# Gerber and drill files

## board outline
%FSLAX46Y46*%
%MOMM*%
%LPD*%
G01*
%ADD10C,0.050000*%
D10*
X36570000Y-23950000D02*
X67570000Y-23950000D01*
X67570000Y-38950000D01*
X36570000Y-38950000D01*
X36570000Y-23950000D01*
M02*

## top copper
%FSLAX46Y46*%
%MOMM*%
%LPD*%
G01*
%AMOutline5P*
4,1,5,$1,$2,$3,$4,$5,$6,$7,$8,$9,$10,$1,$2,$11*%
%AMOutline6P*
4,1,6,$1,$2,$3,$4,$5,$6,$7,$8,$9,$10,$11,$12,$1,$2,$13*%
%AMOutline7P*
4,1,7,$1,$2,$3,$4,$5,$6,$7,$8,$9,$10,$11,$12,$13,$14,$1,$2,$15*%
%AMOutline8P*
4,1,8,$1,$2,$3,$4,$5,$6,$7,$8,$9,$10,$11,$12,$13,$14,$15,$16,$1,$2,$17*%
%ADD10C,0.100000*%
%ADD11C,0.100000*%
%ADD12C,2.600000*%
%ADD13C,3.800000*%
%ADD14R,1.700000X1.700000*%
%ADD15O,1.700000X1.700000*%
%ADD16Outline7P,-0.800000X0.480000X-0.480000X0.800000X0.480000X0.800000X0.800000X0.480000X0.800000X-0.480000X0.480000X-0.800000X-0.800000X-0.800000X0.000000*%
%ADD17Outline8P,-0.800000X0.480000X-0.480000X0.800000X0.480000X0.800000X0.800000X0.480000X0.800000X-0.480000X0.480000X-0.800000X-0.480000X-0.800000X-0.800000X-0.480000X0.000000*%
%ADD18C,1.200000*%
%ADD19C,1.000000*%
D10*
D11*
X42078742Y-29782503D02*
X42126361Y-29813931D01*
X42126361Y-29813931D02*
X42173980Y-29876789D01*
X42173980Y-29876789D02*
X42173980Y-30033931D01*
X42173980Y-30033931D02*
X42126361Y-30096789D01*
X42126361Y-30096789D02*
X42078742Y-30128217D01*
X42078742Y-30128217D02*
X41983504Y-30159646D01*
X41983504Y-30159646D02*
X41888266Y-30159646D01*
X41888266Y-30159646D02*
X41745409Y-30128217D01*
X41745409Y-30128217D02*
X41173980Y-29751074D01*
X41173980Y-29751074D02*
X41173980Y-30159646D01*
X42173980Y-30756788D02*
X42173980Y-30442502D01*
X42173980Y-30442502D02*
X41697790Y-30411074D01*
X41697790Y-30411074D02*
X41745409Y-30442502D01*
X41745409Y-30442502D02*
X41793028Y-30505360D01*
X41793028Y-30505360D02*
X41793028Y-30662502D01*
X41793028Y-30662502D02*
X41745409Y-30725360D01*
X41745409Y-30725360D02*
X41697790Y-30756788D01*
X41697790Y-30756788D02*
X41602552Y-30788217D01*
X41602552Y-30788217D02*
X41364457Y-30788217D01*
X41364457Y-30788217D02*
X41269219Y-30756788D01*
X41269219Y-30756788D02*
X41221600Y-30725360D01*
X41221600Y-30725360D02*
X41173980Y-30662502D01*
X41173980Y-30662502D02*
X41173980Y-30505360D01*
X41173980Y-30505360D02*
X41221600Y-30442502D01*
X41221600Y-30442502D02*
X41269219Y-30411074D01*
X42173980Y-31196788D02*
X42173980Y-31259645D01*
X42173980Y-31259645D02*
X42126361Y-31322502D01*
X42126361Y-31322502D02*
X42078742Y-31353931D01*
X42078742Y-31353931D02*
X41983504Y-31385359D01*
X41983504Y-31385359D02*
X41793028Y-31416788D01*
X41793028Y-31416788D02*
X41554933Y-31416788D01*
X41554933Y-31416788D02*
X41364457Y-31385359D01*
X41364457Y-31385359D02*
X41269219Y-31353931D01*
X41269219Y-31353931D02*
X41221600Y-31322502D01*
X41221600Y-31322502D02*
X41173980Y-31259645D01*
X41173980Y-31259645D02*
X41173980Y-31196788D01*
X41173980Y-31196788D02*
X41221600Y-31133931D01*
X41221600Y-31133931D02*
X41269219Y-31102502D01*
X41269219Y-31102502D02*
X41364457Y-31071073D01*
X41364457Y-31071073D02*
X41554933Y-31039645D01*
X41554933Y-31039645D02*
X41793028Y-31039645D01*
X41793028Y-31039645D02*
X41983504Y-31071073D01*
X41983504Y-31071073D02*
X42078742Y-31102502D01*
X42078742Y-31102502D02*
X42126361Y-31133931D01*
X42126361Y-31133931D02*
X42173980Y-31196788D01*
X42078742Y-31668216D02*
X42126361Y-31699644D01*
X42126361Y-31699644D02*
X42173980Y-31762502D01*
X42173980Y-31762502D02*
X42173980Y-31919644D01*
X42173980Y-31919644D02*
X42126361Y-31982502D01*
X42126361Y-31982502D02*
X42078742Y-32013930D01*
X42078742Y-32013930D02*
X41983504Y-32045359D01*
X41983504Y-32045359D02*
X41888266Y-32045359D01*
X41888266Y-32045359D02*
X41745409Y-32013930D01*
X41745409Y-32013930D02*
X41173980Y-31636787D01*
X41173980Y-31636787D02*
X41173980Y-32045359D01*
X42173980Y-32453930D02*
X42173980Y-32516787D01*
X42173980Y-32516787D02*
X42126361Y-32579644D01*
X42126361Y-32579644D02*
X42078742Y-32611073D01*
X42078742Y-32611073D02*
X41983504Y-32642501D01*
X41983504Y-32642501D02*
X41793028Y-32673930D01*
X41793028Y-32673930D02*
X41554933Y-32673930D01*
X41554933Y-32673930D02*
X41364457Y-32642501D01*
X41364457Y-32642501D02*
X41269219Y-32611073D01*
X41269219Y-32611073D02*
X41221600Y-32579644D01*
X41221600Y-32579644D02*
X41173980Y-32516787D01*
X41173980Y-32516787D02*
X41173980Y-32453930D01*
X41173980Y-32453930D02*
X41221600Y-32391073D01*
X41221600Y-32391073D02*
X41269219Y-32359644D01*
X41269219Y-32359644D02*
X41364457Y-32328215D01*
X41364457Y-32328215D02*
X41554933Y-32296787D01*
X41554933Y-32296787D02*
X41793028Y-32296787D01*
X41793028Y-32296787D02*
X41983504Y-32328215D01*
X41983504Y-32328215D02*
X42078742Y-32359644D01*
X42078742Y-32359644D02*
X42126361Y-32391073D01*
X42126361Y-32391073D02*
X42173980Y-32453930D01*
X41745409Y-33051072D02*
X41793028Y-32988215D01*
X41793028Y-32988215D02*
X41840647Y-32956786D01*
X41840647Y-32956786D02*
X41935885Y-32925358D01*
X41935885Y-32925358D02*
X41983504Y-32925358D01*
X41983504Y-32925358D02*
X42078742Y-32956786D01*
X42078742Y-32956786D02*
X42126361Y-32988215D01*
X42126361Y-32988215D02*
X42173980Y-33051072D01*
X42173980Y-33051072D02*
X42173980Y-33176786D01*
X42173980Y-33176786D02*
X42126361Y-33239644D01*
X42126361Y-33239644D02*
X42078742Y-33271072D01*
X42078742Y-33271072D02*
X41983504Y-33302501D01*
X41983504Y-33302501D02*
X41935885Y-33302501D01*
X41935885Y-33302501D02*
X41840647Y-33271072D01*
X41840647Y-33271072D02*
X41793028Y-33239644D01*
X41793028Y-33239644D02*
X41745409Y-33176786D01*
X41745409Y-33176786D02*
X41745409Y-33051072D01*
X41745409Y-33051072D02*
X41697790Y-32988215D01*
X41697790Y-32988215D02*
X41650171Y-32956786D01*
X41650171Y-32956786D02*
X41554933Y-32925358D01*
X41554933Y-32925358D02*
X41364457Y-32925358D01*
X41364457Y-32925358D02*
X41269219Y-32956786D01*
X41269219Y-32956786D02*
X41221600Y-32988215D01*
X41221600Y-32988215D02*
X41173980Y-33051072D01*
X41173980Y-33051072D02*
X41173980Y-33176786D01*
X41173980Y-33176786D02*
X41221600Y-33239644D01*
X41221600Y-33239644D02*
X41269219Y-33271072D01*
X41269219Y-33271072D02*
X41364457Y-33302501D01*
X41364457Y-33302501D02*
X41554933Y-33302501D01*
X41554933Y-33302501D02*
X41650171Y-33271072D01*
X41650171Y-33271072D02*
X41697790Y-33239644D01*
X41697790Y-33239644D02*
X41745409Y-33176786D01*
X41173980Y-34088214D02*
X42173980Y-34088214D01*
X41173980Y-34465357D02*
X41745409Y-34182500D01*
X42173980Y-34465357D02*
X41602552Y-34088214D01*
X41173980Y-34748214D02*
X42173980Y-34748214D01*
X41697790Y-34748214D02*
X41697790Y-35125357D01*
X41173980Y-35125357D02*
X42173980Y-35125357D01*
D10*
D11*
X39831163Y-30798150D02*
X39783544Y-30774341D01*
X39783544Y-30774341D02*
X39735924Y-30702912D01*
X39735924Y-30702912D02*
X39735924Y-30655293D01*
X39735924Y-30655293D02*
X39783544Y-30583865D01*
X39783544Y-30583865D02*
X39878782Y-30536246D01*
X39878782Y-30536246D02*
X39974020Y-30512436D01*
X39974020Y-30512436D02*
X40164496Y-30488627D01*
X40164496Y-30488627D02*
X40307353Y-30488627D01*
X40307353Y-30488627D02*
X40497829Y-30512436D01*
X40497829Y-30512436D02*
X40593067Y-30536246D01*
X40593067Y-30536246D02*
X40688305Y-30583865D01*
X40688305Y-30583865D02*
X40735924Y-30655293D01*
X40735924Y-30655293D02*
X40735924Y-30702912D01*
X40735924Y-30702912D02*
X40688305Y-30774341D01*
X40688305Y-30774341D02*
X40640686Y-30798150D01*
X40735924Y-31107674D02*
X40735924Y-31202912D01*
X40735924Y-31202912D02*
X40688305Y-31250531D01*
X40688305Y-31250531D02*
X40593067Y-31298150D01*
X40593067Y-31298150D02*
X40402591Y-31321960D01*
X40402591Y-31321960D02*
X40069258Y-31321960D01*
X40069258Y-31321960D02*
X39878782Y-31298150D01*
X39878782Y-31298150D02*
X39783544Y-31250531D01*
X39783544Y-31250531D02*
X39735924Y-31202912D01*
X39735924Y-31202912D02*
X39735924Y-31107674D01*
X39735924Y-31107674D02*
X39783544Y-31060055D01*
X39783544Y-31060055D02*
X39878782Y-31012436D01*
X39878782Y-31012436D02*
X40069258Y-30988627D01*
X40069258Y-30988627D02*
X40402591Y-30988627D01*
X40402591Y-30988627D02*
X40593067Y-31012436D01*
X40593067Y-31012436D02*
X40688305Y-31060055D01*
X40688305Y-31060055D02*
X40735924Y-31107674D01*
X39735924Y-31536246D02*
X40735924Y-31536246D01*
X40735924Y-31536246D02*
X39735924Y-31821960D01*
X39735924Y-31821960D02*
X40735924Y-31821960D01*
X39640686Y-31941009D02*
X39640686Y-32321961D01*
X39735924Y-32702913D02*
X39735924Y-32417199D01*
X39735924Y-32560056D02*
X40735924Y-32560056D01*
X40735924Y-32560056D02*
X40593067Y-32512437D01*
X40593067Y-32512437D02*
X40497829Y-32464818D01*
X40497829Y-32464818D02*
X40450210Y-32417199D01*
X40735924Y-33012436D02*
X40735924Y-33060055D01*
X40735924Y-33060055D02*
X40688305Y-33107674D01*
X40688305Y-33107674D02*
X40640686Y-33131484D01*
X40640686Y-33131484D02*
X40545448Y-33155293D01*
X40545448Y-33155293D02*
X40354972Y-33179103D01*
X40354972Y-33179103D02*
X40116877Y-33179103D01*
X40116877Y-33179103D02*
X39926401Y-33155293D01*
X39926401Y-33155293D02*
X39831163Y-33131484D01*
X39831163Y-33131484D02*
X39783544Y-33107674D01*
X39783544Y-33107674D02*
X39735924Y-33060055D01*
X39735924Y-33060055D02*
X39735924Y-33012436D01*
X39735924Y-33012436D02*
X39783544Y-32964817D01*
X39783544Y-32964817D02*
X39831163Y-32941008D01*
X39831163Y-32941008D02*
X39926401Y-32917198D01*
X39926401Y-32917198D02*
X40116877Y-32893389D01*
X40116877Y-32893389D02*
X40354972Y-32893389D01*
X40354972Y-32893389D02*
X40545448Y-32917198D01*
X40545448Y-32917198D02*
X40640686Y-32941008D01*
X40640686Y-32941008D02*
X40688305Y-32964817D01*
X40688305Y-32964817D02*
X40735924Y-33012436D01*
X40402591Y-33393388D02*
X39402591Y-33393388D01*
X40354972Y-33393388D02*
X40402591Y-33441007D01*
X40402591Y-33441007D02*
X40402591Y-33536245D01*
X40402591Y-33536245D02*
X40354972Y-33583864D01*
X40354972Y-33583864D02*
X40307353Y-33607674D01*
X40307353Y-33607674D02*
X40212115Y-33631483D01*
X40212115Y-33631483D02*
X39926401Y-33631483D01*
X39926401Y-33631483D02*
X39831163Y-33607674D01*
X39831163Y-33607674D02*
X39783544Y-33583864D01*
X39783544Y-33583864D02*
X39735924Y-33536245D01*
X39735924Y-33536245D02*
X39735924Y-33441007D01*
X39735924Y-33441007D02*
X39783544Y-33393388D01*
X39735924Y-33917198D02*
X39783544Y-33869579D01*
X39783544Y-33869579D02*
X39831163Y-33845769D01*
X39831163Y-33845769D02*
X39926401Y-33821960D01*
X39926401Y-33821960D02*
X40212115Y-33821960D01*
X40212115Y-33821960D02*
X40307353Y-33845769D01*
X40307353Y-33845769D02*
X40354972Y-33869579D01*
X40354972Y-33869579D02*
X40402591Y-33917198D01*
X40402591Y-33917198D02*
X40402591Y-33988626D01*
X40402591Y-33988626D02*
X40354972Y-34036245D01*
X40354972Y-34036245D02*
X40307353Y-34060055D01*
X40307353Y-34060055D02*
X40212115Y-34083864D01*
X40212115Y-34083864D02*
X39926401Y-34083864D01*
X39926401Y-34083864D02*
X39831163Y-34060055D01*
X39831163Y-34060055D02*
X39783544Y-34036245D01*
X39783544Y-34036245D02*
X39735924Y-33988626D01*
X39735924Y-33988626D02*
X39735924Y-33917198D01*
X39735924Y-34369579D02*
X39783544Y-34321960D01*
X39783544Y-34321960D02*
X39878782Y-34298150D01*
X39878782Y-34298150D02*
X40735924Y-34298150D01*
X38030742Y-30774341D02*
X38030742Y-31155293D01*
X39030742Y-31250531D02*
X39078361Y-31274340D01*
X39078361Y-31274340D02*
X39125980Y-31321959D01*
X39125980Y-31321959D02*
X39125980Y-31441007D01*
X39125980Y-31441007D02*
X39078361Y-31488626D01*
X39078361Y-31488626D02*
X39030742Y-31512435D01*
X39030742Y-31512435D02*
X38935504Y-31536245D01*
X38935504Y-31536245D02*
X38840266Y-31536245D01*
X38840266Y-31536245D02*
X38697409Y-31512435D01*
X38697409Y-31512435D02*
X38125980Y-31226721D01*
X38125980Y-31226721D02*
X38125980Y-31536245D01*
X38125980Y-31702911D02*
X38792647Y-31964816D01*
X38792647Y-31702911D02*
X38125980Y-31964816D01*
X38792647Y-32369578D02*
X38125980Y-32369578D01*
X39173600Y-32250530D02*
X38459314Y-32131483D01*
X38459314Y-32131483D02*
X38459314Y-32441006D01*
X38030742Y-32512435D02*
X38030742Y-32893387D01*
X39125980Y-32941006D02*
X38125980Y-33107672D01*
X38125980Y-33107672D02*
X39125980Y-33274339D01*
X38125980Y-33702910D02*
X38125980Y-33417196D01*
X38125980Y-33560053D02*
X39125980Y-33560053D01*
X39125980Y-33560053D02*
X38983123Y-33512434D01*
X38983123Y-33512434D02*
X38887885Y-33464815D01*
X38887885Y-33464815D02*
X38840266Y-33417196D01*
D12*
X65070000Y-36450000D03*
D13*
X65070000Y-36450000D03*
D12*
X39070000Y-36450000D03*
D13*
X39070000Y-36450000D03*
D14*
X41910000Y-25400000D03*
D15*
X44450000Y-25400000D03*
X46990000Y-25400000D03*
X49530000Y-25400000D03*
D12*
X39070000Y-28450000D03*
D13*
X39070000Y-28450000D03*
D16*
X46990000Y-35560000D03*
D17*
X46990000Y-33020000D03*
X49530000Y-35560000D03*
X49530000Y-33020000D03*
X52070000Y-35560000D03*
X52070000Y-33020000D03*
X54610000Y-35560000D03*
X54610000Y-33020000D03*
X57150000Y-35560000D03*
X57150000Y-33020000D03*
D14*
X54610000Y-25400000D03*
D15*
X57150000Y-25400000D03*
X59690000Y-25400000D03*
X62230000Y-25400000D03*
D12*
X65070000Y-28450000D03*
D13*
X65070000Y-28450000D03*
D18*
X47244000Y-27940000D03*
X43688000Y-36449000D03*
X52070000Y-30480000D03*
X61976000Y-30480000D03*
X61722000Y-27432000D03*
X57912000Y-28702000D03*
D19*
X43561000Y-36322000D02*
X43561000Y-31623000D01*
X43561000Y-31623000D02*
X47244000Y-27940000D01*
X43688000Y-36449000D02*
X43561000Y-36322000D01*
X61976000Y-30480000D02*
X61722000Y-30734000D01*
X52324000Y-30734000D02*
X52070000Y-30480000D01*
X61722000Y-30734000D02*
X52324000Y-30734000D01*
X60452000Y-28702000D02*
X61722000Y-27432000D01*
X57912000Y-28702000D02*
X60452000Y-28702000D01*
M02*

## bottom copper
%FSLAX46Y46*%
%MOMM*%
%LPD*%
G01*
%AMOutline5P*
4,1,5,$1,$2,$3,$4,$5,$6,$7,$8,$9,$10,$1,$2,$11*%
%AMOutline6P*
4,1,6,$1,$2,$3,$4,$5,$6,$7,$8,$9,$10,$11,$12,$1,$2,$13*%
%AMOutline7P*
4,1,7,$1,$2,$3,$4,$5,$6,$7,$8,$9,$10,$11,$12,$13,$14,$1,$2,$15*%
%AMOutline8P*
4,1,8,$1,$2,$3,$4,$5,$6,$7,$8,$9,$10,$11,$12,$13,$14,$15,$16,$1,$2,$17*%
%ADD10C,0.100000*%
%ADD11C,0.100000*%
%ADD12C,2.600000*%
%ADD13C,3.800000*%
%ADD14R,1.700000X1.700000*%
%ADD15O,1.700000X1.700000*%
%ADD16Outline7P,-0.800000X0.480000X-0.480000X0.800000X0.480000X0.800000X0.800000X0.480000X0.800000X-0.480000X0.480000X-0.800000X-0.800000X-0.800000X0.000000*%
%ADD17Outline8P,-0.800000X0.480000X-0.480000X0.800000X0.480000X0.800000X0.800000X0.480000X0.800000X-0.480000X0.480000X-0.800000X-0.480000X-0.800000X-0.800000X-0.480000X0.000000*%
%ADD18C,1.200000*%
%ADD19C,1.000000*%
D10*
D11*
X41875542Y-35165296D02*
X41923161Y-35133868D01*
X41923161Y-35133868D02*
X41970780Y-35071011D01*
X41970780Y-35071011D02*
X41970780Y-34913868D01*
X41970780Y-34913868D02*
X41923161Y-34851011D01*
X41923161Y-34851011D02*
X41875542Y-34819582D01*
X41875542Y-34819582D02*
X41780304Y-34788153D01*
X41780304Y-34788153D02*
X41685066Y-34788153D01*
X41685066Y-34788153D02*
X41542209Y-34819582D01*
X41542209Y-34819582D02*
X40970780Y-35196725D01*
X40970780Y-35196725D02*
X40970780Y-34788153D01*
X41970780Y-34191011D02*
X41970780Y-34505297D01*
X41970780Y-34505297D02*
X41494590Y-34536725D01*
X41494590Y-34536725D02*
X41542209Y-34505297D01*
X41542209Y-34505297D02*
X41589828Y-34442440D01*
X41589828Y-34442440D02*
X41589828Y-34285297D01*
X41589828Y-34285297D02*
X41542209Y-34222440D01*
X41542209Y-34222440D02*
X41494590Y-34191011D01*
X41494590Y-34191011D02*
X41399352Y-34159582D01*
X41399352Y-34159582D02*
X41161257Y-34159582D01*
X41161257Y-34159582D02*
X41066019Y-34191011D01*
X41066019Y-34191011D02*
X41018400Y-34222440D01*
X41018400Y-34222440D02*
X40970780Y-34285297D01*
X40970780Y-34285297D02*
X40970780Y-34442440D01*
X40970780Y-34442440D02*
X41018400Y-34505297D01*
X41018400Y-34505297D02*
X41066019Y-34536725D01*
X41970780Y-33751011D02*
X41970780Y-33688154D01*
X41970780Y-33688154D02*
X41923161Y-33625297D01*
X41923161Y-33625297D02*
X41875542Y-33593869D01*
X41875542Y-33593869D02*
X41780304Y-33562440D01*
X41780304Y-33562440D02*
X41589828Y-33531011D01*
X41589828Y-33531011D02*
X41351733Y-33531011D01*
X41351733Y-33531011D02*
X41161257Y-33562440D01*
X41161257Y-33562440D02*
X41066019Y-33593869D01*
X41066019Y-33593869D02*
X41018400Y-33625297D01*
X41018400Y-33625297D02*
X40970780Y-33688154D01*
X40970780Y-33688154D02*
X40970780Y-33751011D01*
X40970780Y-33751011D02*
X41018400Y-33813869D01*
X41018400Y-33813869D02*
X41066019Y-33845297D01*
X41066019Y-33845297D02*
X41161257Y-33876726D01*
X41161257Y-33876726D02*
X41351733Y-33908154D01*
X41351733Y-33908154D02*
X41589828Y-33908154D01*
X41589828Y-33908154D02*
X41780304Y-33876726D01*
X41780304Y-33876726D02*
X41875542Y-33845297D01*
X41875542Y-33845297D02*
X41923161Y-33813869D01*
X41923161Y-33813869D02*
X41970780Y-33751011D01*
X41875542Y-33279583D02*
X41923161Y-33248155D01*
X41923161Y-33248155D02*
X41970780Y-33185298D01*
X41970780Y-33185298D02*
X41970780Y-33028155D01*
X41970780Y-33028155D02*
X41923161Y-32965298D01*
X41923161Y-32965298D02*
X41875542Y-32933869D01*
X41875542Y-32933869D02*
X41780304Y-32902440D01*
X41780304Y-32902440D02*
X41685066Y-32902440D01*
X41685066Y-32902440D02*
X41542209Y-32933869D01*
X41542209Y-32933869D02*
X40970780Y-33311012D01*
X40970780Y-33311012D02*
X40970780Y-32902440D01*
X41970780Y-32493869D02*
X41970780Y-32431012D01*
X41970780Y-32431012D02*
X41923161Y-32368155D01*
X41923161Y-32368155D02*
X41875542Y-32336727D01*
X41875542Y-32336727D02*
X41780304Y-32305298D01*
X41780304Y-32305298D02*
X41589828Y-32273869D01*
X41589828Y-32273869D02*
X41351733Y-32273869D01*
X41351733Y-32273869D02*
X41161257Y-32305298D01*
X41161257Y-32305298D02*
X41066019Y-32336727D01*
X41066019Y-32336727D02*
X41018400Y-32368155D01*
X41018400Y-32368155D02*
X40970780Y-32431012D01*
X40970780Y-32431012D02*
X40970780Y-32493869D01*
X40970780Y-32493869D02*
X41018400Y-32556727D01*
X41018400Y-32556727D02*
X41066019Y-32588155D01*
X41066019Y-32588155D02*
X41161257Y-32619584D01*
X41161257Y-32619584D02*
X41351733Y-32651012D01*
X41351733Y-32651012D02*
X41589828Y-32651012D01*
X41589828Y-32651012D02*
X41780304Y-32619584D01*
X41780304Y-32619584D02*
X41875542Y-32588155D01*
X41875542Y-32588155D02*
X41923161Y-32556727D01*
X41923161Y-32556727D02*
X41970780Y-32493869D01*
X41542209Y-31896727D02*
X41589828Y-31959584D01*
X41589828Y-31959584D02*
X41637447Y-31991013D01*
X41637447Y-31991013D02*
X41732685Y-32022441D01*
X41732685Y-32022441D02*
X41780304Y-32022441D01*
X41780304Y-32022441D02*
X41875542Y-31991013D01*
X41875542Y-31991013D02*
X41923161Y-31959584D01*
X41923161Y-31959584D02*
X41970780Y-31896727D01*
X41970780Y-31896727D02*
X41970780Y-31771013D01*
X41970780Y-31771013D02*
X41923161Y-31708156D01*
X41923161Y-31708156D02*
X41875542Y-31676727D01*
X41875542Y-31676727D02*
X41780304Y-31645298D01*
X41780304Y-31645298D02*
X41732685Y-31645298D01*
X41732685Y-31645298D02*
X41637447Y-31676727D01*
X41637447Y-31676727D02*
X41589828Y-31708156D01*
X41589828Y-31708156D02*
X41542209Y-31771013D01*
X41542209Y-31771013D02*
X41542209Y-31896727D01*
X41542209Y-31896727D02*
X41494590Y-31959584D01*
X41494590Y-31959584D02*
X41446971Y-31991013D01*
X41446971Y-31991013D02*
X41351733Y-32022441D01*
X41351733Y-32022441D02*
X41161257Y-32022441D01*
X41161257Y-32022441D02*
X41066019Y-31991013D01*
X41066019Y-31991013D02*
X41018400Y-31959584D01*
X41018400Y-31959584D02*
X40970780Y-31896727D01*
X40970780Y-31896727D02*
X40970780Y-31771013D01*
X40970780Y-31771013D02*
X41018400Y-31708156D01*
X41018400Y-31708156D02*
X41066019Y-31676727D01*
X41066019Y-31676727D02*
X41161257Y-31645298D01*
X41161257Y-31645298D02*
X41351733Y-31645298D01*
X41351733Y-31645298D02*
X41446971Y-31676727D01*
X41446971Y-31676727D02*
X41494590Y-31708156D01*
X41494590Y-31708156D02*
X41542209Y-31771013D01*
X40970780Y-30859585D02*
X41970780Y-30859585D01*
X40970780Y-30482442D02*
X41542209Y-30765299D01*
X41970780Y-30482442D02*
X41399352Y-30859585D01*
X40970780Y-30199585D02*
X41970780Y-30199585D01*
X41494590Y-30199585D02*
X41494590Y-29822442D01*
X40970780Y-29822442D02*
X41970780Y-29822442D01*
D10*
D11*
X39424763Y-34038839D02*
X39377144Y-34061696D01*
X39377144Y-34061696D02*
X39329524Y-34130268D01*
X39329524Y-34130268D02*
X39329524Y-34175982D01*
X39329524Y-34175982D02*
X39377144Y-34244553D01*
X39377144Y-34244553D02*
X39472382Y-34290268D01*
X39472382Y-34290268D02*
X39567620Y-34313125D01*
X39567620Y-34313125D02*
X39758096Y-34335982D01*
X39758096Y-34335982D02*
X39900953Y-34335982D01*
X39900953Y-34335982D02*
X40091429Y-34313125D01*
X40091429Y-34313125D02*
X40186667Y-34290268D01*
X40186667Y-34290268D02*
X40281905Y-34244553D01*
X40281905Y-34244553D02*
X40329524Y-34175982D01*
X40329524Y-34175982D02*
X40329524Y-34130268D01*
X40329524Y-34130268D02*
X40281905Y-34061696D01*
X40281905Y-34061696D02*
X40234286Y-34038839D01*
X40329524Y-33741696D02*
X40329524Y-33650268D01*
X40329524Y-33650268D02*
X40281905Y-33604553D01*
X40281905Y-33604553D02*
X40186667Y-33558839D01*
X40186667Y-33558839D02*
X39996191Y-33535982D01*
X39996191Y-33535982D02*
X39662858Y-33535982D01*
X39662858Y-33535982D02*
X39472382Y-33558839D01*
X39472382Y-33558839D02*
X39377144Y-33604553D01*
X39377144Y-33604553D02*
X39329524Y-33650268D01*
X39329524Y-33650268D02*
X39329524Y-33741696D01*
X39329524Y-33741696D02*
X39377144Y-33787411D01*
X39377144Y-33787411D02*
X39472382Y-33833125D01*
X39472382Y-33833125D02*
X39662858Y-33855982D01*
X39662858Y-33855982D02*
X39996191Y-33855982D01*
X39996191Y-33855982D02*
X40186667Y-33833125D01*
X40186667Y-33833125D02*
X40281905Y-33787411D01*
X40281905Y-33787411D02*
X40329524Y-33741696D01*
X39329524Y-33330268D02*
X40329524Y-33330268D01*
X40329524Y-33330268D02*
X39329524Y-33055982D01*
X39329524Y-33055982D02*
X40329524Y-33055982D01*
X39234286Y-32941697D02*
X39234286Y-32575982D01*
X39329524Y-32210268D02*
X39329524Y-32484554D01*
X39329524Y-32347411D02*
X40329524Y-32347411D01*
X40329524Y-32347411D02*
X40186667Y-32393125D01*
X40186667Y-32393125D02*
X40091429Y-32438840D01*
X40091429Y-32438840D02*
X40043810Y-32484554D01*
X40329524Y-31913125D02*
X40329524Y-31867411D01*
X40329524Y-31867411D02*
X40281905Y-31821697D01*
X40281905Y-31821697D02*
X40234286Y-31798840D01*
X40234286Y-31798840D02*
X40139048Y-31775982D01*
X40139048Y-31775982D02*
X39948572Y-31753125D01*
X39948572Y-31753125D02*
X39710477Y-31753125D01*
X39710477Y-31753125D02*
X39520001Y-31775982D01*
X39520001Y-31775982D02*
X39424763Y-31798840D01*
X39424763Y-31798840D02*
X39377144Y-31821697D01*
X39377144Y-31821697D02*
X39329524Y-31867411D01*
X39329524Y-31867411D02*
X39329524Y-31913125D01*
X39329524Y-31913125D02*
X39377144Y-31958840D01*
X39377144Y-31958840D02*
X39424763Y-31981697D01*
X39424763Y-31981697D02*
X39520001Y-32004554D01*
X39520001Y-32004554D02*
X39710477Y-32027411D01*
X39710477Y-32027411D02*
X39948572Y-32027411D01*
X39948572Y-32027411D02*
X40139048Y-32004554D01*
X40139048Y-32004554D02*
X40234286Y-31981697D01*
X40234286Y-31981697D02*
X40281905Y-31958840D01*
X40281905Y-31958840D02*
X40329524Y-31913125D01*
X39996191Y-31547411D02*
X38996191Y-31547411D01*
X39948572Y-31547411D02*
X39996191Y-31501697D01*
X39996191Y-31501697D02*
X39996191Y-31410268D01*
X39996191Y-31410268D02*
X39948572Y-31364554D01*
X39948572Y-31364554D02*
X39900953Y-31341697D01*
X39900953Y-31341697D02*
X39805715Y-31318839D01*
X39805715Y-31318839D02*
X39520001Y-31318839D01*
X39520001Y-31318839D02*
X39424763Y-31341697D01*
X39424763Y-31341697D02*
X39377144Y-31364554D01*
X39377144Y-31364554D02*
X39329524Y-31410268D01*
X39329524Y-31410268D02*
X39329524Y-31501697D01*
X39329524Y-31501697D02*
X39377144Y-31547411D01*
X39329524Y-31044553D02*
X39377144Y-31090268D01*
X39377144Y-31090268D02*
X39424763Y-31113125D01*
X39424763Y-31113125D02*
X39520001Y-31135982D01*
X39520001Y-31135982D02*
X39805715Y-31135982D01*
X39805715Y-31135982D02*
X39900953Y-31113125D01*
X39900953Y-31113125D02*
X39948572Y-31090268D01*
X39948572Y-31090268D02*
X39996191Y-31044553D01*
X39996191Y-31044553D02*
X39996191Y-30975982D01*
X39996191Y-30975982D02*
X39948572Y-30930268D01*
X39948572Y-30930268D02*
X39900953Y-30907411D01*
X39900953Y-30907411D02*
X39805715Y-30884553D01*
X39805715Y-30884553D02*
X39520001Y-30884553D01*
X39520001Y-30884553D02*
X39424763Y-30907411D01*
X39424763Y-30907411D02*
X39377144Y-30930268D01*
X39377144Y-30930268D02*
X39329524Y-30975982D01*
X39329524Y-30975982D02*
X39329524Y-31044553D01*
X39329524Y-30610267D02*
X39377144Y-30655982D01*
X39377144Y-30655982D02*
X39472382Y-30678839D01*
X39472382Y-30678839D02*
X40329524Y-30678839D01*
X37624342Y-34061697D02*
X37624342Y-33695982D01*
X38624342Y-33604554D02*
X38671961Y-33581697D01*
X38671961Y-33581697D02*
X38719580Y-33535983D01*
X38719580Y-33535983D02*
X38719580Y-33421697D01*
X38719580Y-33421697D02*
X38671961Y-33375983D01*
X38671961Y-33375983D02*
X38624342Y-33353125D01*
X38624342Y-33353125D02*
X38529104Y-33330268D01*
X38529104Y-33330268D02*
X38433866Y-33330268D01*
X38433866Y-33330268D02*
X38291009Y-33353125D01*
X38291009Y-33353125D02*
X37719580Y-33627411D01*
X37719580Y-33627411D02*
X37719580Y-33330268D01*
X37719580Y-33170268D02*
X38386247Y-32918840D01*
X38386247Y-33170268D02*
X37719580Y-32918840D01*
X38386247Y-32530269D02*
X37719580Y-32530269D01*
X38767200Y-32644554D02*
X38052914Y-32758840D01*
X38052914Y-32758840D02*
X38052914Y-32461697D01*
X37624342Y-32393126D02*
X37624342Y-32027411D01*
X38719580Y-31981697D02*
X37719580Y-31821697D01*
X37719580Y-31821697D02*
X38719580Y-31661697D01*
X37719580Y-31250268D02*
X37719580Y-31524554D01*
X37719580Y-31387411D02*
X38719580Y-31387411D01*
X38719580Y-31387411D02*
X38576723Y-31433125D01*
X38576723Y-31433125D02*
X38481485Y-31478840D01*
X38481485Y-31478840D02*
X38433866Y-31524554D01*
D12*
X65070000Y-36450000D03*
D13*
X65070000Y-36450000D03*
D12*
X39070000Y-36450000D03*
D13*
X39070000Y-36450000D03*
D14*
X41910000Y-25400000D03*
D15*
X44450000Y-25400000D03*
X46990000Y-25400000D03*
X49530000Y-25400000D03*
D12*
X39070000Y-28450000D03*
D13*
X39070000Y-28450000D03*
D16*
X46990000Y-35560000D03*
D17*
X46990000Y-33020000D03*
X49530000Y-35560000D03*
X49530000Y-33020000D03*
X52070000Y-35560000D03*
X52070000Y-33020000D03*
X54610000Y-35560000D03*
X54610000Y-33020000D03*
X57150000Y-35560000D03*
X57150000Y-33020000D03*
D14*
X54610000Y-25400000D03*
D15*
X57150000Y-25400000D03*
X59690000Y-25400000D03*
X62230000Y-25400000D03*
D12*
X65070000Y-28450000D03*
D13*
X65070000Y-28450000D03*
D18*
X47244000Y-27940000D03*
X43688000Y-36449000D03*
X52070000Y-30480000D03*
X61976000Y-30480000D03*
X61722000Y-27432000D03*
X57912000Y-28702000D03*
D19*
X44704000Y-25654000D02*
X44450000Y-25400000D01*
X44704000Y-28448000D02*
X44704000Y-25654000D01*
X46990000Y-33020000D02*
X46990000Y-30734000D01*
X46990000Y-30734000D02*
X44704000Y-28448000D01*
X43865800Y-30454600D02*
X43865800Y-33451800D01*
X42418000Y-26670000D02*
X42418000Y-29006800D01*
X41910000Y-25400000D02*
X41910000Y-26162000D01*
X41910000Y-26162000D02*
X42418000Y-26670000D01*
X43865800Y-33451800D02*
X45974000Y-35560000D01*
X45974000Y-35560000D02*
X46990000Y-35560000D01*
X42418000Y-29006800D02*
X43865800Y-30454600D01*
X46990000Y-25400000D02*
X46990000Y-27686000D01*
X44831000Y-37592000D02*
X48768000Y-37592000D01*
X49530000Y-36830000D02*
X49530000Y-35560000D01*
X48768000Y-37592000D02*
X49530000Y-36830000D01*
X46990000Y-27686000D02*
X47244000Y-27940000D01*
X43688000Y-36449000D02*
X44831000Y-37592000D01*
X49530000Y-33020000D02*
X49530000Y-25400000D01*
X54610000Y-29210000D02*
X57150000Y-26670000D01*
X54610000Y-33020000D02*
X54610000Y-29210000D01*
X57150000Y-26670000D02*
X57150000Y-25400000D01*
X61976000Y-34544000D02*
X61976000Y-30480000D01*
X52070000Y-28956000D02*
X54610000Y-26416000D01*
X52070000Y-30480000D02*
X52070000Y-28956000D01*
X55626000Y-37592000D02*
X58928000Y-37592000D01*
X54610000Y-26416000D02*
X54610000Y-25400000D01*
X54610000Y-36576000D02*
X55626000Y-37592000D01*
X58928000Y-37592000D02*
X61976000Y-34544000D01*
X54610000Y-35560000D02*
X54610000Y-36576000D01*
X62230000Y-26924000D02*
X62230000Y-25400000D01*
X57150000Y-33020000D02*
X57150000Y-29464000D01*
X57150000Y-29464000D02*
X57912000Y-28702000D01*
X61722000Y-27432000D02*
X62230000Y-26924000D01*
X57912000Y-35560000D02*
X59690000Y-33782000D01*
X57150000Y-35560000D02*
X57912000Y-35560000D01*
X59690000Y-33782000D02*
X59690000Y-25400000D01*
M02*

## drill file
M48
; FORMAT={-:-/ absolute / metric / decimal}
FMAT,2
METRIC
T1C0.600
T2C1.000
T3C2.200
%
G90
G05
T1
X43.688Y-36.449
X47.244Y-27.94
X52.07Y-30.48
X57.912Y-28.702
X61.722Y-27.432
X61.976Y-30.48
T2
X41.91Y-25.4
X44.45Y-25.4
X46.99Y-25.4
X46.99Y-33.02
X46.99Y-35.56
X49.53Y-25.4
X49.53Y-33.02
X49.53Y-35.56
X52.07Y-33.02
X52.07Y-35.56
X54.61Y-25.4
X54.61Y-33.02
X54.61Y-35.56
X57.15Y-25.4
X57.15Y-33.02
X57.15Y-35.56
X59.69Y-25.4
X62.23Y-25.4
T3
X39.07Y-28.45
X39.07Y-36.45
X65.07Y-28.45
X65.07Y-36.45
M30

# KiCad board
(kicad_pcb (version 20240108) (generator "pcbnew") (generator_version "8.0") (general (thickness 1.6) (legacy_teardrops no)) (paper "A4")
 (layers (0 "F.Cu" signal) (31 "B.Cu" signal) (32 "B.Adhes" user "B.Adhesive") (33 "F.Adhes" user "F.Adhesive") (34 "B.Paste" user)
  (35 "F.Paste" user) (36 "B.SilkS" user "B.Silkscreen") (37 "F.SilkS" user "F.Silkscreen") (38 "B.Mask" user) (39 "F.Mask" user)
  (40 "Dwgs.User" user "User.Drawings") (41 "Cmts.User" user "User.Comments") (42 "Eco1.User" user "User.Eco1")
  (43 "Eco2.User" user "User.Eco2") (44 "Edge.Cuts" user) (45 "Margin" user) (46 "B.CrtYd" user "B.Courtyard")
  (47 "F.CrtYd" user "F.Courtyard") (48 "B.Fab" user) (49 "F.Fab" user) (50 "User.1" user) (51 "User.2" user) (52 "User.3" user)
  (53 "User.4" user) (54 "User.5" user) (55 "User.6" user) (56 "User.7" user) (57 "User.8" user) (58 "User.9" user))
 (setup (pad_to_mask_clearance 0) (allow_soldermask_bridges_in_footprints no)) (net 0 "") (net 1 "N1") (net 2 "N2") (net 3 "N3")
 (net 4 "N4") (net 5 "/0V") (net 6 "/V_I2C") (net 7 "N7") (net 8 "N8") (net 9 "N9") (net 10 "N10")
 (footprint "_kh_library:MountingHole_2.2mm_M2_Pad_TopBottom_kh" (layer "F.Cu") (at 65.07 36.45)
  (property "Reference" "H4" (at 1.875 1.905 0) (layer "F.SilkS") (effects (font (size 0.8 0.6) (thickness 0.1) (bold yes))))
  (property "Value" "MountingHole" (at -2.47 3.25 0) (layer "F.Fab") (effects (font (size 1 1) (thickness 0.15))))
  (pad "1" thru_hole circle (at 0 0) (size 2.6 2.6) (drill 2.2) (layers "*.Cu" "*.Mask") (remove_unused_layers no))
  (pad "1" connect circle (at 0 0) (size 3.8 3.8) (layers "F.Cu" "F.Mask"))
  (pad "1" connect circle (at 0 0) (size 3.8 3.8) (layers "B.Cu" "B.Mask")))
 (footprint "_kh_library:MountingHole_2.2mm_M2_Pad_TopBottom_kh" (layer "F.Cu") (at 39.07 36.45)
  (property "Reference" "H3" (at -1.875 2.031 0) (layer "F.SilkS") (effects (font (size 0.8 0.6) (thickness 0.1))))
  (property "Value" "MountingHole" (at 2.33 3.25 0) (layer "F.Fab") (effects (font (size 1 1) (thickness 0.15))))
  (pad "1" thru_hole circle (at 0 0) (size 2.6 2.6) (drill 2.2) (layers "*.Cu" "*.Mask") (remove_unused_layers no))
  (pad "1" connect circle (at 0 0) (size 3.8 3.8) (layers "F.Cu" "F.Mask"))
  (pad "1" connect circle (at 0 0) (size 3.8 3.8) (layers "B.Cu" "B.Mask")))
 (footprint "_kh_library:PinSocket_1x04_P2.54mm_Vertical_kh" (layer "F.Cu") (at 41.91 25.4 90)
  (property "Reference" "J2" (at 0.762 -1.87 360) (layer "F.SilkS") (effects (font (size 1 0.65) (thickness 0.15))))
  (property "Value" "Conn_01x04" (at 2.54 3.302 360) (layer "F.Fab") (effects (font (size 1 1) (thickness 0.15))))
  (pad "1" thru_hole rect (at 0 0 90) (size 1.7 1.7) (drill 1) (layers "*.Cu" "*.Mask") (remove_unused_layers no) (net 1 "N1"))
  (pad "2" thru_hole oval (at 0 2.54 90) (size 1.7 1.7) (drill 1) (layers "*.Cu" "*.Mask") (remove_unused_layers no) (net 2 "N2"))
  (pad "3" thru_hole oval (at 0 5.08 90) (size 1.7 1.7) (drill 1) (layers "*.Cu" "*.Mask") (remove_unused_layers no) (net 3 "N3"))
  (pad "4" thru_hole oval (at 0 7.62 90) (size 1.7 1.7) (drill 1) (layers "*.Cu" "*.Mask") (remove_unused_layers no) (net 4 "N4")))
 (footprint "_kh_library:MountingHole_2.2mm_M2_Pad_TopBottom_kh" (layer "F.Cu") (at 39.07 28.45)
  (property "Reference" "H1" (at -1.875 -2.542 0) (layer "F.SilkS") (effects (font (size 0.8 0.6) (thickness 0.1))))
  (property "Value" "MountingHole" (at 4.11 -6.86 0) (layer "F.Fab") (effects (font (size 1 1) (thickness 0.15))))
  (pad "1" thru_hole circle (at 0 0) (size 2.6 2.6) (drill 2.2) (layers "*.Cu" "*.Mask") (remove_unused_layers no))
  (pad "1" connect circle (at 0 0) (size 3.8 3.8) (layers "F.Cu" "F.Mask"))
  (pad "1" connect circle (at 0 0) (size 3.8 3.8) (layers "B.Cu" "B.Mask")))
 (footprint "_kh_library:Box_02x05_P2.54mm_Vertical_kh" (layer "F.Cu") (at 46.99 35.56)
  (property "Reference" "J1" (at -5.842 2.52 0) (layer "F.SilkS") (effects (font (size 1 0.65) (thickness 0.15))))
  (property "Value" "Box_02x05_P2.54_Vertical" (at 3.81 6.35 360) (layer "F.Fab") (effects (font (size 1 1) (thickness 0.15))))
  (pad "1" thru_hole roundrect (at 0 0) (size 1.6 1.6) (drill 1) (layers "*.Cu" "*.Mask") (remove_unused_layers no) (roundrect_rratio 0)
   (chamfer_ratio 0.2) (chamfer top_left top_right bottom_right) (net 1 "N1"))
  (pad "2" thru_hole roundrect (at 0 -2.54) (size 1.6 1.6) (drill 1) (layers "*.Cu" "*.Mask") (remove_unused_layers no) (roundrect_rratio 0)
   (chamfer_ratio 0.2) (chamfer top_left top_right bottom_left bottom_right) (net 2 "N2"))
  (pad "3" thru_hole roundrect (at 2.54 0) (size 1.6 1.6) (drill 1) (layers "*.Cu" "*.Mask") (remove_unused_layers no) (roundrect_rratio 0)
   (chamfer_ratio 0.2) (chamfer top_left top_right bottom_left bottom_right) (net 3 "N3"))
  (pad "4" thru_hole roundrect (at 2.54 -2.54) (size 1.6 1.6) (drill 1) (layers "*.Cu" "*.Mask") (remove_unused_layers no)
   (roundrect_rratio 0) (chamfer_ratio 0.2) (chamfer top_left top_right bottom_left bottom_right) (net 4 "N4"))
  (pad "5" thru_hole roundrect (at 5.08 0) (size 1.6 1.6) (drill 1) (layers "*.Cu" "*.Mask") (remove_unused_layers no) (roundrect_rratio 0)
   (chamfer_ratio 0.2) (chamfer top_left top_right bottom_left bottom_right) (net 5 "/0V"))
  (pad "6" thru_hole roundrect (at 5.08 -2.54) (size 1.6 1.6) (drill 1) (layers "*.Cu" "*.Mask") (remove_unused_layers no)
   (roundrect_rratio 0) (chamfer_ratio 0.2) (chamfer top_left top_right bottom_left bottom_right) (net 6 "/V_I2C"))
  (pad "7" thru_hole roundrect (at 7.62 0) (size 1.6 1.6) (drill 1) (layers "*.Cu" "*.Mask") (remove_unused_layers no) (roundrect_rratio 0)
   (chamfer_ratio 0.2) (chamfer top_left top_right bottom_left bottom_right) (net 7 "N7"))
  (pad "8" thru_hole roundrect (at 7.62 -2.54) (size 1.6 1.6) (drill 1) (layers "*.Cu" "*.Mask") (remove_unused_layers no)
   (roundrect_rratio 0) (chamfer_ratio 0.2) (chamfer top_left top_right bottom_left bottom_right) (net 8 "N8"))
  (pad "9" thru_hole roundrect (at 10.16 0) (size 1.6 1.6) (drill 1) (layers "*.Cu" "*.Mask") (remove_unused_layers no) (roundrect_rratio 0)
   (chamfer_ratio 0.2) (chamfer top_left top_right bottom_left bottom_right) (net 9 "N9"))
  (pad "10" thru_hole roundrect (at 10.16 -2.54) (size 1.6 1.6) (drill 1) (layers "*.Cu" "*.Mask") (remove_unused_layers no)
   (roundrect_rratio 0) (chamfer_ratio 0.2) (chamfer top_left top_right bottom_left bottom_right) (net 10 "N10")))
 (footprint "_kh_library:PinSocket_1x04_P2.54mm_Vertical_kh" (layer "F.Cu") (at 54.61 25.4 90)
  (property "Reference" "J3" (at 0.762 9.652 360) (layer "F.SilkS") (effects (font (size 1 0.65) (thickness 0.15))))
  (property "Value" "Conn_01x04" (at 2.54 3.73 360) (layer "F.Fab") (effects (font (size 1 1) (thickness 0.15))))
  (pad "1" thru_hole rect (at 0 0 90) (size 1.7 1.7) (drill 1) (layers "*.Cu" "*.Mask") (remove_unused_layers no) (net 7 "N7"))
  (pad "2" thru_hole oval (at 0 2.54 90) (size 1.7 1.7) (drill 1) (layers "*.Cu" "*.Mask") (remove_unused_layers no) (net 8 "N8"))
  (pad "3" thru_hole oval (at 0 5.08 90) (size 1.7 1.7) (drill 1) (layers "*.Cu" "*.Mask") (remove_unused_layers no) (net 9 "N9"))
  (pad "4" thru_hole oval (at 0 7.62 90) (size 1.7 1.7) (drill 1) (layers "*.Cu" "*.Mask") (remove_unused_layers no) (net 10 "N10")))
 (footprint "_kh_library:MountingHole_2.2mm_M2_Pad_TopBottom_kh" (layer "F.Cu") (at 65.07 28.45)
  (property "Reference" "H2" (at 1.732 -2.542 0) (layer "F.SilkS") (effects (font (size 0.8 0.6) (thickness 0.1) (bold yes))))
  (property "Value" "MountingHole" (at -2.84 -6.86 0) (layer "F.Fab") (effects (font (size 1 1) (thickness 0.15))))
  (pad "1" thru_hole circle (at 0 0) (size 2.6 2.6) (drill 2.2) (layers "*.Cu" "*.Mask") (remove_unused_layers no))
  (pad "1" connect circle (at 0 0) (size 3.8 3.8) (layers "F.Cu" "F.Mask"))
  (pad "1" connect circle (at 0 0) (size 3.8 3.8) (layers "B.Cu" "B.Mask")))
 (gr_rect (start 36.57 23.95) (end 67.57 38.95) (stroke (width 0.05) (type default)) (fill none) (layer "Edge.Cuts"))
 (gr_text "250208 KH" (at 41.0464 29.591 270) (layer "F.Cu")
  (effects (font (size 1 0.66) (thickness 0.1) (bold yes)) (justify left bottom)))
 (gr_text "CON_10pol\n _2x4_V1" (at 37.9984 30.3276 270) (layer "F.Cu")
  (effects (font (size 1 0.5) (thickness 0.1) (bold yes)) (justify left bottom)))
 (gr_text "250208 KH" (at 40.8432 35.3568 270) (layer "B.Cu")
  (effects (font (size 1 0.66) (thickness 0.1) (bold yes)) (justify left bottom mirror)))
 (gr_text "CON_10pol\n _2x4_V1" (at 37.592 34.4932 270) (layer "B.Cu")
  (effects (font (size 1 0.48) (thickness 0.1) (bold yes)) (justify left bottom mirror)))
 (segment (start 44.704 25.654) (end 44.45 25.4) (width 1) (layer "B.Cu") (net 2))
 (segment (start 44.704 28.448) (end 44.704 25.654) (width 1) (layer "B.Cu") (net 2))
 (segment (start 46.99 33.02) (end 46.99 30.734) (width 1) (layer "B.Cu") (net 2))
 (segment (start 46.99 30.734) (end 44.704 28.448) (width 1) (layer "B.Cu") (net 2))
 (segment (start 43.8658 30.4546) (end 43.8658 33.4518) (width 1) (layer "B.Cu") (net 1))
 (segment (start 42.418 26.67) (end 42.418 29.0068) (width 1) (layer "B.Cu") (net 1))
 (segment (start 41.91 25.4) (end 41.91 26.162) (width 1) (layer "B.Cu") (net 1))
 (segment (start 41.91 26.162) (end 42.418 26.67) (width 1) (layer "B.Cu") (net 1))
 (segment (start 43.8658 33.4518) (end 45.974 35.56) (width 1) (layer "B.Cu") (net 1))
 (segment (start 45.974 35.56) (end 46.99 35.56) (width 1) (layer "B.Cu") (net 1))
 (segment (start 42.418 29.0068) (end 43.8658 30.4546) (width 1) (layer "B.Cu") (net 1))
 (segment (start 43.561 36.322) (end 43.561 31.623) (width 1) (layer "F.Cu") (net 3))
 (segment (start 43.561 31.623) (end 47.244 27.94) (width 1) (layer "F.Cu") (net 3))
 (segment (start 43.688 36.449) (end 43.561 36.322) (width 1) (layer "F.Cu") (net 3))
 (via (at 47.244 27.94) (size 1.2) (drill 0.6) (layers "F.Cu" "B.Cu") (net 3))
 (via (at 43.688 36.449) (size 1.2) (drill 0.6) (layers "F.Cu" "B.Cu") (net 3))
 (segment (start 46.99 25.4) (end 46.99 27.686) (width 1) (layer "B.Cu") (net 3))
 (segment (start 44.831 37.592) (end 48.768 37.592) (width 1) (layer "B.Cu") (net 3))
 (segment (start 49.53 36.83) (end 49.53 35.56) (width 1) (layer "B.Cu") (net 3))
 (segment (start 48.768 37.592) (end 49.53 36.83) (width 1) (layer "B.Cu") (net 3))
 (segment (start 46.99 27.686) (end 47.244 27.94) (width 1) (layer "B.Cu") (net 3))
 (segment (start 43.688 36.449) (end 44.831 37.592) (width 1) (layer "B.Cu") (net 3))
 (segment (start 49.53 33.02) (end 49.53 25.4) (width 1) (layer "B.Cu") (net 4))
 (segment (start 54.61 29.21) (end 57.15 26.67) (width 1) (layer "B.Cu") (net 8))
 (segment (start 54.61 33.02) (end 54.61 29.21) (width 1) (layer "B.Cu") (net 8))
 (segment (start 57.15 26.67) (end 57.15 25.4) (width 1) (layer "B.Cu") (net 8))
 (segment (start 61.976 30.48) (end 61.722 30.734) (width 1) (layer "F.Cu") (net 7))
 (segment (start 52.324 30.734) (end 52.07 30.48) (width 1) (layer "F.Cu") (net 7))
 (segment (start 61.722 30.734) (end 52.324 30.734) (width 1) (layer "F.Cu") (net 7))
 (via (at 52.07 30.48) (size 1.2) (drill 0.6) (layers "F.Cu" "B.Cu") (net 7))
 (via (at 61.976 30.48) (size 1.2) (drill 0.6) (layers "F.Cu" "B.Cu") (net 7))
 (segment (start 61.976 34.544) (end 61.976 30.48) (width 1) (layer "B.Cu") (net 7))
 (segment (start 52.07 28.956) (end 54.61 26.416) (width 1) (layer "B.Cu") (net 7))
 (segment (start 52.07 30.48) (end 52.07 28.956) (width 1) (layer "B.Cu") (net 7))
 (segment (start 55.626 37.592) (end 58.928 37.592) (width 1) (layer "B.Cu") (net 7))
 (segment (start 54.61 26.416) (end 54.61 25.4) (width 1) (layer "B.Cu") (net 7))
 (segment (start 54.61 36.576) (end 55.626 37.592) (width 1) (layer "B.Cu") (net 7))
 (segment (start 58.928 37.592) (end 61.976 34.544) (width 1) (layer "B.Cu") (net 7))
 (segment (start 54.61 35.56) (end 54.61 36.576) (width 1) (layer "B.Cu") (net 7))
 (segment (start 60.452 28.702) (end 61.722 27.432) (width 1) (layer "F.Cu") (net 10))
 (segment (start 57.912 28.702) (end 60.452 28.702) (width 1) (layer "F.Cu") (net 10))
 (via (at 61.722 27.432) (size 1.2) (drill 0.6) (layers "F.Cu" "B.Cu") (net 10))
 (via (at 57.912 28.702) (size 1.2) (drill 0.6) (layers "F.Cu" "B.Cu") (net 10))
 (segment (start 62.23 26.924) (end 62.23 25.4) (width 1) (layer "B.Cu") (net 10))
 (segment (start 57.15 33.02) (end 57.15 29.464) (width 1) (layer "B.Cu") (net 10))
 (segment (start 57.15 29.464) (end 57.912 28.702) (width 1) (layer "B.Cu") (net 10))
 (segment (start 61.722 27.432) (end 62.23 26.924) (width 1) (layer "B.Cu") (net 10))
 (segment (start 57.912 35.56) (end 59.69 33.782) (width 1) (layer "B.Cu") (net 9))
 (segment (start 57.15 35.56) (end 57.912 35.56) (width 1) (layer "B.Cu") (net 9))
 (segment (start 59.69 33.782) (end 59.69 25.4) (width 1) (layer "B.Cu") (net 9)))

